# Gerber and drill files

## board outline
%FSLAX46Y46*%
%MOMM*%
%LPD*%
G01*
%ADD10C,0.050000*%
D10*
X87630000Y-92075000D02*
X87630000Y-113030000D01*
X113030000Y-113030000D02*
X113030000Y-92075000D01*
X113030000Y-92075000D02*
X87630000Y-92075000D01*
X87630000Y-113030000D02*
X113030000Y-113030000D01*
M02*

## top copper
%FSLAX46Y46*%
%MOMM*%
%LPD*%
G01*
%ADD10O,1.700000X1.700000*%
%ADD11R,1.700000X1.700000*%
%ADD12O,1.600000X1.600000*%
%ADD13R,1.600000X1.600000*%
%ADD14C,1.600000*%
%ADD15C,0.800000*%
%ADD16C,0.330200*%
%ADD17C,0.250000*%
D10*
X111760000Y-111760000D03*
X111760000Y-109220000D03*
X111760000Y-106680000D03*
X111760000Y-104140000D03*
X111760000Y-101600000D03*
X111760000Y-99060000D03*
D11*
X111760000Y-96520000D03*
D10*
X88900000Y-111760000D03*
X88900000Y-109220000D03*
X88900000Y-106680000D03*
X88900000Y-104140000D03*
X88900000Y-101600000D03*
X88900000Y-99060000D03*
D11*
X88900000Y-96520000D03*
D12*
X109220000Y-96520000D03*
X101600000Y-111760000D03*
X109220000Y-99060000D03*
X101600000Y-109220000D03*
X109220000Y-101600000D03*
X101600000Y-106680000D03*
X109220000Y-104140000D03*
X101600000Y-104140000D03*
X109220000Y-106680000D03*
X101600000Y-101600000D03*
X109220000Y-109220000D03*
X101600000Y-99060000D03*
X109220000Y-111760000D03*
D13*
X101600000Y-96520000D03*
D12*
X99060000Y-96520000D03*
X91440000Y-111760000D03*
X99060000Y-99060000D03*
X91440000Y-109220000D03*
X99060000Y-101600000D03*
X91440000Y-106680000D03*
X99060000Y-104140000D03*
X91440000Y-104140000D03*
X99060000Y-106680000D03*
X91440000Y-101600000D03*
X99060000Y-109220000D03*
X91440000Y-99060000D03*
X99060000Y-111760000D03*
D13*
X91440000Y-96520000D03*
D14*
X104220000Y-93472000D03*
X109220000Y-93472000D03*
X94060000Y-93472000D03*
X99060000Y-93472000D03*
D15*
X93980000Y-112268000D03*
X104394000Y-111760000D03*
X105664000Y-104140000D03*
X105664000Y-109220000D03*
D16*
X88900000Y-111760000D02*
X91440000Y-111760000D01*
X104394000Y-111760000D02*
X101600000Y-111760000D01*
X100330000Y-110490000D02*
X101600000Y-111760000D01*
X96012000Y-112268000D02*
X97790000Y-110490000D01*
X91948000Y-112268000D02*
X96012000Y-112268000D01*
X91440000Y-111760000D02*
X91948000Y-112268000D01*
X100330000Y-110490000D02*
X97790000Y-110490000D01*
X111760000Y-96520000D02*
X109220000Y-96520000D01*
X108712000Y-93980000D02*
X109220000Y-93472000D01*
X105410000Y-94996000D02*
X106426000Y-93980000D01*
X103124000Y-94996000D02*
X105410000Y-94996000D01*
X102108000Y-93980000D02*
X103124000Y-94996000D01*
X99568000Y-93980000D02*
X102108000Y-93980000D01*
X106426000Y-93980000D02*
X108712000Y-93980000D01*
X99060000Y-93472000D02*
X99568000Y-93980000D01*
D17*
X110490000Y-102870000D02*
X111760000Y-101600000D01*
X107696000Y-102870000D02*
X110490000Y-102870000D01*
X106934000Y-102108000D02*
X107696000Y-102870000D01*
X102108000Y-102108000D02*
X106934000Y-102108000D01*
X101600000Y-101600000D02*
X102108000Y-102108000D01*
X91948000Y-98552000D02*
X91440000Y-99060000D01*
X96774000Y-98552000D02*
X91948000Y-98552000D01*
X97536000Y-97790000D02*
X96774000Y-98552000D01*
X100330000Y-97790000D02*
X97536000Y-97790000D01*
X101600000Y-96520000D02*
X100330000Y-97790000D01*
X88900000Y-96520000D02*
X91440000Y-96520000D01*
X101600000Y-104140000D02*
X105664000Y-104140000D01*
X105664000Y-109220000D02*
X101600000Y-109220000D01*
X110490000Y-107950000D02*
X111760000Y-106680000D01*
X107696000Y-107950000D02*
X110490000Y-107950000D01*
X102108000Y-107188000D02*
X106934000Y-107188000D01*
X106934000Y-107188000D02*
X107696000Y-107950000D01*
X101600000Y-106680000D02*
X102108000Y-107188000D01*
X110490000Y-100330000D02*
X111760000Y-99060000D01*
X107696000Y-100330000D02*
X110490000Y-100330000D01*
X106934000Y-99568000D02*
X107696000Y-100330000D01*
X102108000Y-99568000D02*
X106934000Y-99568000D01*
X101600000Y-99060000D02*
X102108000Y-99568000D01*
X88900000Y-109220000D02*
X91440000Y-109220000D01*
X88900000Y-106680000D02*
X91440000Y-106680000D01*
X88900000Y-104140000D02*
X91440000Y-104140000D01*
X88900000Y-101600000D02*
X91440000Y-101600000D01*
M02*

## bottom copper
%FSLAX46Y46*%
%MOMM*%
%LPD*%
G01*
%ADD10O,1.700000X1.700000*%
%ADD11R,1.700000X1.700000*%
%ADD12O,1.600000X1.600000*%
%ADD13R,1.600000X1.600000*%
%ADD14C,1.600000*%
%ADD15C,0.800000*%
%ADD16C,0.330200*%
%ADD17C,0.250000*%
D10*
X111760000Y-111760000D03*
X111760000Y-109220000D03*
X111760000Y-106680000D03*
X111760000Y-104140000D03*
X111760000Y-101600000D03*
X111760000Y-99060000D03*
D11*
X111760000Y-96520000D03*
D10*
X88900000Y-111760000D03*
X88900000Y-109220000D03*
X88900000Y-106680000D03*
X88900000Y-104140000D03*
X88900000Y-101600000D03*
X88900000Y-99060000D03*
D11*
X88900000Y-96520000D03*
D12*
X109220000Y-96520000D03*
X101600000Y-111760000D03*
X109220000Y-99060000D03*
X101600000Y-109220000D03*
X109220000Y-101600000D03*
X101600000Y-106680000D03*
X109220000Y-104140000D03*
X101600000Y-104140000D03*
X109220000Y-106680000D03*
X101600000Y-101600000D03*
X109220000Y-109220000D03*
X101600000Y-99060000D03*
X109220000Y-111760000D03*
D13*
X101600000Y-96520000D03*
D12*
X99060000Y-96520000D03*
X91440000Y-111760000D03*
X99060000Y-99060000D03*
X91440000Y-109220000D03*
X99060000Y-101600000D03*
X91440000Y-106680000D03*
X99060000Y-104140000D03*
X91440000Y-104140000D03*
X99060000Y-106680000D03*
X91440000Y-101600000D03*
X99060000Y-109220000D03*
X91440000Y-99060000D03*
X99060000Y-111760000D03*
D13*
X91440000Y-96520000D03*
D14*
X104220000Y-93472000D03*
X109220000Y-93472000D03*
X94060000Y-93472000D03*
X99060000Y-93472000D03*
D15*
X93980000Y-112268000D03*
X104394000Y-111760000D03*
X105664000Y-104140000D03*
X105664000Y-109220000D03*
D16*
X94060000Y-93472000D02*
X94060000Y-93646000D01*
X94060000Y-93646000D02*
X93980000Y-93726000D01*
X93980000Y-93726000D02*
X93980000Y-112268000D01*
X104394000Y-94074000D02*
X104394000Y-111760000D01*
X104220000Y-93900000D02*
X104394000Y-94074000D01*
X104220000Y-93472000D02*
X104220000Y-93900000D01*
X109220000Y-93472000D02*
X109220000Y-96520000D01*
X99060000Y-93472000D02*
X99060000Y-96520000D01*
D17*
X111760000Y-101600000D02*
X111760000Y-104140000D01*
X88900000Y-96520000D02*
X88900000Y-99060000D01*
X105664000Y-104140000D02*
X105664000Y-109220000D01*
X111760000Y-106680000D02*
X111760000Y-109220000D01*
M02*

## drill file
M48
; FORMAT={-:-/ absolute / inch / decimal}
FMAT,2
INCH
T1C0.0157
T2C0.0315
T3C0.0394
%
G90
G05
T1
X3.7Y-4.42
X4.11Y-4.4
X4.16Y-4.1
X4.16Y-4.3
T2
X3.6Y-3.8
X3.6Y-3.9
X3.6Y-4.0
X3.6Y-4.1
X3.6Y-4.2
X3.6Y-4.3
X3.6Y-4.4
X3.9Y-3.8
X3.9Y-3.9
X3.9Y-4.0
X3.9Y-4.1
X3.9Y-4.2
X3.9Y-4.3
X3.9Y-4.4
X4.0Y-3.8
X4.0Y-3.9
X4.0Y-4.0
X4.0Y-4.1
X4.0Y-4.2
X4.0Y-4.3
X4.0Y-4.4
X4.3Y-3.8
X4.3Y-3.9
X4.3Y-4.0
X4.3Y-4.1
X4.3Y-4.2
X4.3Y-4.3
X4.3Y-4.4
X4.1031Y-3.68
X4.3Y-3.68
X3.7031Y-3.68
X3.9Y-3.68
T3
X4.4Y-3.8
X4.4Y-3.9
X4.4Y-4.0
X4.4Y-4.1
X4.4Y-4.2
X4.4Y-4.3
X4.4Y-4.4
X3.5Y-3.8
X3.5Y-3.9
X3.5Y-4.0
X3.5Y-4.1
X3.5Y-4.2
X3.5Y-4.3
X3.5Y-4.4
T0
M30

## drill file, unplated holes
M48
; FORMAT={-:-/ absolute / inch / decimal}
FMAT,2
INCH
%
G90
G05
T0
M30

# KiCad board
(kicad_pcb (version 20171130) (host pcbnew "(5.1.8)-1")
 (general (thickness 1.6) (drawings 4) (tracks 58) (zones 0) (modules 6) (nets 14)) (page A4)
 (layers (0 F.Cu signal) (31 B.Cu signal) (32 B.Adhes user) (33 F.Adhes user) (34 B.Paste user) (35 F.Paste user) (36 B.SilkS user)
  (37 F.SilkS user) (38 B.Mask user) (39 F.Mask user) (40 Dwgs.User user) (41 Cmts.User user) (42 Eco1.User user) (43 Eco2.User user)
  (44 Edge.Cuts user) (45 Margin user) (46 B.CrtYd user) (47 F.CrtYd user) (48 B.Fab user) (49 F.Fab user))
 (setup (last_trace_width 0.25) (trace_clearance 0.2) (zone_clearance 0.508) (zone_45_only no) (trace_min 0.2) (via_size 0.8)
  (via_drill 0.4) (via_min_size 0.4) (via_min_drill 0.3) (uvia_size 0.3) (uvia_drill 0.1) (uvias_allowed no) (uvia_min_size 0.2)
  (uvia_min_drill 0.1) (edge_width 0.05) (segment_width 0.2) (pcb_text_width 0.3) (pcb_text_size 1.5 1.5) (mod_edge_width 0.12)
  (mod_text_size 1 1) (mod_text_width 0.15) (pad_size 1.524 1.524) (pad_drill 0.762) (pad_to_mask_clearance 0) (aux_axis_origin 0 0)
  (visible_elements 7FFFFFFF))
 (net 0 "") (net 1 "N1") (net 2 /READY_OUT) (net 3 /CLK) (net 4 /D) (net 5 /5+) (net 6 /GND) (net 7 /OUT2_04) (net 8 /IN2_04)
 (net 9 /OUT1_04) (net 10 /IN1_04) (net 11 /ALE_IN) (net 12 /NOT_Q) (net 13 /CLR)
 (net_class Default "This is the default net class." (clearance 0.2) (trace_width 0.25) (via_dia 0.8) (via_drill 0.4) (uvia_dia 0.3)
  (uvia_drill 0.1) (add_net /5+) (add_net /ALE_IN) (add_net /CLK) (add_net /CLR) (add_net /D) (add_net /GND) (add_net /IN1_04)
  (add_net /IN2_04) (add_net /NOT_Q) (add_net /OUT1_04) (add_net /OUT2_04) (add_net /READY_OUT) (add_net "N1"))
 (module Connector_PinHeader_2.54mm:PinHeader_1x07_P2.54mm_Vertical (layer F.Cu) (at 111.76 96.52)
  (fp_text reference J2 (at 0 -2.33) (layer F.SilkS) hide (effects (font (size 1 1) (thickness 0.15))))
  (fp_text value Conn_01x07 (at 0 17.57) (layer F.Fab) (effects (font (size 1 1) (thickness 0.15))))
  (pad 7 thru_hole oval (at 0 15.24) (size 1.7 1.7) (drill 1) (layers *.Cu *.Mask) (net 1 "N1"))
  (pad 6 thru_hole oval (at 0 12.7) (size 1.7 1.7) (drill 1) (layers *.Cu *.Mask) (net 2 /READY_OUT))
  (pad 5 thru_hole oval (at 0 10.16) (size 1.7 1.7) (drill 1) (layers *.Cu *.Mask) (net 2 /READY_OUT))
  (pad 4 thru_hole oval (at 0 7.62) (size 1.7 1.7) (drill 1) (layers *.Cu *.Mask) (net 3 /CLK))
  (pad 3 thru_hole oval (at 0 5.08) (size 1.7 1.7) (drill 1) (layers *.Cu *.Mask) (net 3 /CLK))
  (pad 2 thru_hole oval (at 0 2.54) (size 1.7 1.7) (drill 1) (layers *.Cu *.Mask) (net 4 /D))
  (pad 1 thru_hole rect (at 0 0) (size 1.7 1.7) (drill 1) (layers *.Cu *.Mask) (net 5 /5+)))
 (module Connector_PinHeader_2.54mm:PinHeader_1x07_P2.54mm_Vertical (layer F.Cu) (at 88.9 96.52)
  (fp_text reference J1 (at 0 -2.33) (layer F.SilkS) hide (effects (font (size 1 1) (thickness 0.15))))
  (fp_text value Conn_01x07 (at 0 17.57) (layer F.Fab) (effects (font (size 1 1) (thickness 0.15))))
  (pad 7 thru_hole oval (at 0 15.24) (size 1.7 1.7) (drill 1) (layers *.Cu *.Mask) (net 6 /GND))
  (pad 6 thru_hole oval (at 0 12.7) (size 1.7 1.7) (drill 1) (layers *.Cu *.Mask) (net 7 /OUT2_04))
  (pad 5 thru_hole oval (at 0 10.16) (size 1.7 1.7) (drill 1) (layers *.Cu *.Mask) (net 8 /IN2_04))
  (pad 4 thru_hole oval (at 0 7.62) (size 1.7 1.7) (drill 1) (layers *.Cu *.Mask) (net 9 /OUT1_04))
  (pad 3 thru_hole oval (at 0 5.08) (size 1.7 1.7) (drill 1) (layers *.Cu *.Mask) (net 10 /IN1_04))
  (pad 2 thru_hole oval (at 0 2.54) (size 1.7 1.7) (drill 1) (layers *.Cu *.Mask) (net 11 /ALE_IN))
  (pad 1 thru_hole rect (at 0 0) (size 1.7 1.7) (drill 1) (layers *.Cu *.Mask) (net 11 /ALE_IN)))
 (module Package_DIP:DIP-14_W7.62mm (layer F.Cu) (at 101.6 96.52)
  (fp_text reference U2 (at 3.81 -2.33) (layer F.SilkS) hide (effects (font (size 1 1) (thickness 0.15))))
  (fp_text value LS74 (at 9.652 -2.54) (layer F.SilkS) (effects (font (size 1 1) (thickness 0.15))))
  (pad 14 thru_hole oval (at 7.62 0) (size 1.6 1.6) (drill 0.8) (layers *.Cu *.Mask) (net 5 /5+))
  (pad 7 thru_hole oval (at 0 15.24) (size 1.6 1.6) (drill 0.8) (layers *.Cu *.Mask) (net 6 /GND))
  (pad 13 thru_hole oval (at 7.62 2.54) (size 1.6 1.6) (drill 0.8) (layers *.Cu *.Mask))
  (pad 6 thru_hole oval (at 0 12.7) (size 1.6 1.6) (drill 0.8) (layers *.Cu *.Mask) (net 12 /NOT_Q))
  (pad 12 thru_hole oval (at 7.62 5.08) (size 1.6 1.6) (drill 0.8) (layers *.Cu *.Mask))
  (pad 5 thru_hole oval (at 0 10.16) (size 1.6 1.6) (drill 0.8) (layers *.Cu *.Mask) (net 2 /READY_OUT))
  (pad 11 thru_hole oval (at 7.62 7.62) (size 1.6 1.6) (drill 0.8) (layers *.Cu *.Mask))
  (pad 4 thru_hole oval (at 0 7.62) (size 1.6 1.6) (drill 0.8) (layers *.Cu *.Mask) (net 12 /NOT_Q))
  (pad 10 thru_hole oval (at 7.62 10.16) (size 1.6 1.6) (drill 0.8) (layers *.Cu *.Mask))
  (pad 3 thru_hole oval (at 0 5.08) (size 1.6 1.6) (drill 0.8) (layers *.Cu *.Mask) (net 3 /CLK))
  (pad 9 thru_hole oval (at 7.62 12.7) (size 1.6 1.6) (drill 0.8) (layers *.Cu *.Mask))
  (pad 2 thru_hole oval (at 0 2.54) (size 1.6 1.6) (drill 0.8) (layers *.Cu *.Mask) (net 4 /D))
  (pad 8 thru_hole oval (at 7.62 15.24) (size 1.6 1.6) (drill 0.8) (layers *.Cu *.Mask))
  (pad 1 thru_hole rect (at 0 0) (size 1.6 1.6) (drill 0.8) (layers *.Cu *.Mask) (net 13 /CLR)))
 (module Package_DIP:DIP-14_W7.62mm (layer F.Cu) (at 91.44 96.52)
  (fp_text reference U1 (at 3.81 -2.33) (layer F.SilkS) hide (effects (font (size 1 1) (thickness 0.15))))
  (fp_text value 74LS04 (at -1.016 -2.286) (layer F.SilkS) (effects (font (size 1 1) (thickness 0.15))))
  (pad 14 thru_hole oval (at 7.62 0) (size 1.6 1.6) (drill 0.8) (layers *.Cu *.Mask) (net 5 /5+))
  (pad 7 thru_hole oval (at 0 15.24) (size 1.6 1.6) (drill 0.8) (layers *.Cu *.Mask) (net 6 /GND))
  (pad 13 thru_hole oval (at 7.62 2.54) (size 1.6 1.6) (drill 0.8) (layers *.Cu *.Mask))
  (pad 6 thru_hole oval (at 0 12.7) (size 1.6 1.6) (drill 0.8) (layers *.Cu *.Mask) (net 7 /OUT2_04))
  (pad 12 thru_hole oval (at 7.62 5.08) (size 1.6 1.6) (drill 0.8) (layers *.Cu *.Mask))
  (pad 5 thru_hole oval (at 0 10.16) (size 1.6 1.6) (drill 0.8) (layers *.Cu *.Mask) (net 8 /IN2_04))
  (pad 11 thru_hole oval (at 7.62 7.62) (size 1.6 1.6) (drill 0.8) (layers *.Cu *.Mask))
  (pad 4 thru_hole oval (at 0 7.62) (size 1.6 1.6) (drill 0.8) (layers *.Cu *.Mask) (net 9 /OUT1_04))
  (pad 10 thru_hole oval (at 7.62 10.16) (size 1.6 1.6) (drill 0.8) (layers *.Cu *.Mask))
  (pad 3 thru_hole oval (at 0 5.08) (size 1.6 1.6) (drill 0.8) (layers *.Cu *.Mask) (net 10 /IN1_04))
  (pad 9 thru_hole oval (at 7.62 12.7) (size 1.6 1.6) (drill 0.8) (layers *.Cu *.Mask))
  (pad 2 thru_hole oval (at 0 2.54) (size 1.6 1.6) (drill 0.8) (layers *.Cu *.Mask) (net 13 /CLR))
  (pad 8 thru_hole oval (at 7.62 15.24) (size 1.6 1.6) (drill 0.8) (layers *.Cu *.Mask))
  (pad 1 thru_hole rect (at 0 0) (size 1.6 1.6) (drill 0.8) (layers *.Cu *.Mask) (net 11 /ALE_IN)))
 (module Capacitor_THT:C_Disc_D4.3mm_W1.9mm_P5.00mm (layer F.Cu) (at 109.22 93.472 180)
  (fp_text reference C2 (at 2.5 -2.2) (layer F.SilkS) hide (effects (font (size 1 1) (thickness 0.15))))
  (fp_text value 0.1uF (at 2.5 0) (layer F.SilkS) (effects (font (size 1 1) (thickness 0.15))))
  (pad 2 thru_hole circle (at 5 0 180) (size 1.6 1.6) (drill 0.8) (layers *.Cu *.Mask) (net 6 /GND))
  (pad 1 thru_hole circle (at 0 0 180) (size 1.6 1.6) (drill 0.8) (layers *.Cu *.Mask) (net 5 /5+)))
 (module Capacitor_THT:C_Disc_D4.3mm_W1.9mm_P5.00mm (layer F.Cu) (at 99.06 93.472 180)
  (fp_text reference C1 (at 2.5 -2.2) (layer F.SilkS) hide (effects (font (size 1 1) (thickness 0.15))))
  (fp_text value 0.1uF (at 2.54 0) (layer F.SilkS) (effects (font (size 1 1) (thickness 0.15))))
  (pad 2 thru_hole circle (at 5 0 180) (size 1.6 1.6) (drill 0.8) (layers *.Cu *.Mask) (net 6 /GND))
  (pad 1 thru_hole circle (at 0 0 180) (size 1.6 1.6) (drill 0.8) (layers *.Cu *.Mask) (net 5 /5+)))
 (gr_line (start 87.63 92.075) (end 87.63 113.03) (layer Edge.Cuts) (width 0.05))
 (gr_line (start 113.03 113.03) (end 113.03 92.075) (layer Edge.Cuts) (width 0.05))
 (gr_line (start 113.03 92.075) (end 87.63 92.075) (layer Edge.Cuts) (width 0.05))
 (gr_line (start 87.63 113.03) (end 113.03 113.03) (layer Edge.Cuts) (width 0.05))
 (segment (start 88.9 111.76) (end 91.44 111.76) (width 0.3302) (layer F.Cu) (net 6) (status 30))
 (segment (start 94.06 93.472) (end 94.06 93.646) (width 0.3302) (layer B.Cu) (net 6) (status 30))
 (segment (start 94.06 93.646) (end 93.98 93.726) (width 0.3302) (layer B.Cu) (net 6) (status 30))
 (segment (start 93.98 93.726) (end 93.98 112.268) (width 0.3302) (layer B.Cu) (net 6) (status 10))
 (via (at 93.98 112.268) (size 0.8) (drill 0.4) (layers F.Cu B.Cu) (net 6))
 (segment (start 104.394 94.074) (end 104.394 111.76) (width 0.3302) (layer B.Cu) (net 6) (status 10))
 (segment (start 104.22 93.9) (end 104.394 94.074) (width 0.3302) (layer B.Cu) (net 6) (status 30))
 (segment (start 104.22 93.472) (end 104.22 93.9) (width 0.3302) (layer B.Cu) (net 6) (status 30))
 (via (at 104.394 111.76) (size 0.8) (drill 0.4) (layers F.Cu B.Cu) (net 6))
 (segment (start 104.394 111.76) (end 101.6 111.76) (width 0.3302) (layer F.Cu) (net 6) (status 20))
 (segment (start 100.33 110.49) (end 101.6 111.76) (width 0.3302) (layer F.Cu) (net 6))
 (segment (start 96.012 112.268) (end 97.79 110.49) (width 0.3302) (layer F.Cu) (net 6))
 (segment (start 91.948 112.268) (end 96.012 112.268) (width 0.3302) (layer F.Cu) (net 6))
 (segment (start 91.44 111.76) (end 91.948 112.268) (width 0.3302) (layer F.Cu) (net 6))
 (segment (start 100.33 110.49) (end 97.79 110.49) (width 0.3302) (layer F.Cu) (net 6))
 (segment (start 111.76 96.52) (end 109.22 96.52) (width 0.3302) (layer F.Cu) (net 5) (status 30))
 (segment (start 109.22 93.472) (end 109.22 96.52) (width 0.3302) (layer B.Cu) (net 5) (status 30))
 (segment (start 99.06 93.472) (end 99.06 96.52) (width 0.3302) (layer B.Cu) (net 5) (status 30))
 (segment (start 108.712 93.98) (end 109.22 93.472) (width 0.3302) (layer F.Cu) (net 5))
 (segment (start 105.41 94.996) (end 106.426 93.98) (width 0.3302) (layer F.Cu) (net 5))
 (segment (start 103.124 94.996) (end 105.41 94.996) (width 0.3302) (layer F.Cu) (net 5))
 (segment (start 102.108 93.98) (end 103.124 94.996) (width 0.3302) (layer F.Cu) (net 5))
 (segment (start 99.568 93.98) (end 102.108 93.98) (width 0.3302) (layer F.Cu) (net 5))
 (segment (start 106.426 93.98) (end 108.712 93.98) (width 0.3302) (layer F.Cu) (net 5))
 (segment (start 99.06 93.472) (end 99.568 93.98) (width 0.3302) (layer F.Cu) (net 5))
 (segment (start 111.76 101.6) (end 111.76 104.14) (width 0.25) (layer B.Cu) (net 3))
 (segment (start 110.49 102.87) (end 111.76 101.6) (width 0.25) (layer F.Cu) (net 3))
 (segment (start 107.696 102.87) (end 110.49 102.87) (width 0.25) (layer F.Cu) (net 3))
 (segment (start 106.934 102.108) (end 107.696 102.87) (width 0.25) (layer F.Cu) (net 3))
 (segment (start 102.108 102.108) (end 106.934 102.108) (width 0.25) (layer F.Cu) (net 3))
 (segment (start 101.6 101.6) (end 102.108 102.108) (width 0.25) (layer F.Cu) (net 3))
 (segment (start 91.948 98.552) (end 91.44 99.06) (width 0.25) (layer F.Cu) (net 13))
 (segment (start 96.774 98.552) (end 91.948 98.552) (width 0.25) (layer F.Cu) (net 13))
 (segment (start 97.536 97.79) (end 96.774 98.552) (width 0.25) (layer F.Cu) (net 13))
 (segment (start 100.33 97.79) (end 97.536 97.79) (width 0.25) (layer F.Cu) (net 13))
 (segment (start 101.6 96.52) (end 100.33 97.79) (width 0.25) (layer F.Cu) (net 13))
 (segment (start 88.9 96.52) (end 91.44 96.52) (width 0.25) (layer F.Cu) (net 11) (status 30))
 (segment (start 88.9 96.52) (end 88.9 99.06) (width 0.25) (layer B.Cu) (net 11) (status 30))
 (segment (start 101.6 104.14) (end 105.664 104.14) (width 0.25) (layer F.Cu) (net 12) (status 10))
 (via (at 105.664 104.14) (size 0.8) (drill 0.4) (layers F.Cu B.Cu) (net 12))
 (segment (start 105.664 104.14) (end 105.664 109.22) (width 0.25) (layer B.Cu) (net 12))
 (via (at 105.664 109.22) (size 0.8) (drill 0.4) (layers F.Cu B.Cu) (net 12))
 (segment (start 105.664 109.22) (end 101.6 109.22) (width 0.25) (layer F.Cu) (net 12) (status 20))
 (segment (start 111.76 106.68) (end 111.76 109.22) (width 0.25) (layer B.Cu) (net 2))
 (segment (start 110.49 107.95) (end 111.76 106.68) (width 0.25) (layer F.Cu) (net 2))
 (segment (start 107.696 107.95) (end 110.49 107.95) (width 0.25) (layer F.Cu) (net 2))
 (segment (start 102.108 107.188) (end 106.934 107.188) (width 0.25) (layer F.Cu) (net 2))
 (segment (start 106.934 107.188) (end 107.696 107.95) (width 0.25) (layer F.Cu) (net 2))
 (segment (start 101.6 106.68) (end 102.108 107.188) (width 0.25) (layer F.Cu) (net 2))
 (segment (start 110.49 100.33) (end 111.76 99.06) (width 0.25) (layer F.Cu) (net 4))
 (segment (start 107.696 100.33) (end 110.49 100.33) (width 0.25) (layer F.Cu) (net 4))
 (segment (start 106.934 99.568) (end 107.696 100.33) (width 0.25) (layer F.Cu) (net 4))
 (segment (start 102.108 99.568) (end 106.934 99.568) (width 0.25) (layer F.Cu) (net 4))
 (segment (start 101.6 99.06) (end 102.108 99.568) (width 0.25) (layer F.Cu) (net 4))
 (segment (start 88.9 109.22) (end 91.44 109.22) (width 0.25) (layer F.Cu) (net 7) (status 30))
 (segment (start 88.9 106.68) (end 91.44 106.68) (width 0.25) (layer F.Cu) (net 8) (status 30))
 (segment (start 88.9 104.14) (end 91.44 104.14) (width 0.25) (layer F.Cu) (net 9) (status 30))
 (segment (start 88.9 101.6) (end 91.44 101.6) (width 0.25) (layer F.Cu) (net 10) (status 30)))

